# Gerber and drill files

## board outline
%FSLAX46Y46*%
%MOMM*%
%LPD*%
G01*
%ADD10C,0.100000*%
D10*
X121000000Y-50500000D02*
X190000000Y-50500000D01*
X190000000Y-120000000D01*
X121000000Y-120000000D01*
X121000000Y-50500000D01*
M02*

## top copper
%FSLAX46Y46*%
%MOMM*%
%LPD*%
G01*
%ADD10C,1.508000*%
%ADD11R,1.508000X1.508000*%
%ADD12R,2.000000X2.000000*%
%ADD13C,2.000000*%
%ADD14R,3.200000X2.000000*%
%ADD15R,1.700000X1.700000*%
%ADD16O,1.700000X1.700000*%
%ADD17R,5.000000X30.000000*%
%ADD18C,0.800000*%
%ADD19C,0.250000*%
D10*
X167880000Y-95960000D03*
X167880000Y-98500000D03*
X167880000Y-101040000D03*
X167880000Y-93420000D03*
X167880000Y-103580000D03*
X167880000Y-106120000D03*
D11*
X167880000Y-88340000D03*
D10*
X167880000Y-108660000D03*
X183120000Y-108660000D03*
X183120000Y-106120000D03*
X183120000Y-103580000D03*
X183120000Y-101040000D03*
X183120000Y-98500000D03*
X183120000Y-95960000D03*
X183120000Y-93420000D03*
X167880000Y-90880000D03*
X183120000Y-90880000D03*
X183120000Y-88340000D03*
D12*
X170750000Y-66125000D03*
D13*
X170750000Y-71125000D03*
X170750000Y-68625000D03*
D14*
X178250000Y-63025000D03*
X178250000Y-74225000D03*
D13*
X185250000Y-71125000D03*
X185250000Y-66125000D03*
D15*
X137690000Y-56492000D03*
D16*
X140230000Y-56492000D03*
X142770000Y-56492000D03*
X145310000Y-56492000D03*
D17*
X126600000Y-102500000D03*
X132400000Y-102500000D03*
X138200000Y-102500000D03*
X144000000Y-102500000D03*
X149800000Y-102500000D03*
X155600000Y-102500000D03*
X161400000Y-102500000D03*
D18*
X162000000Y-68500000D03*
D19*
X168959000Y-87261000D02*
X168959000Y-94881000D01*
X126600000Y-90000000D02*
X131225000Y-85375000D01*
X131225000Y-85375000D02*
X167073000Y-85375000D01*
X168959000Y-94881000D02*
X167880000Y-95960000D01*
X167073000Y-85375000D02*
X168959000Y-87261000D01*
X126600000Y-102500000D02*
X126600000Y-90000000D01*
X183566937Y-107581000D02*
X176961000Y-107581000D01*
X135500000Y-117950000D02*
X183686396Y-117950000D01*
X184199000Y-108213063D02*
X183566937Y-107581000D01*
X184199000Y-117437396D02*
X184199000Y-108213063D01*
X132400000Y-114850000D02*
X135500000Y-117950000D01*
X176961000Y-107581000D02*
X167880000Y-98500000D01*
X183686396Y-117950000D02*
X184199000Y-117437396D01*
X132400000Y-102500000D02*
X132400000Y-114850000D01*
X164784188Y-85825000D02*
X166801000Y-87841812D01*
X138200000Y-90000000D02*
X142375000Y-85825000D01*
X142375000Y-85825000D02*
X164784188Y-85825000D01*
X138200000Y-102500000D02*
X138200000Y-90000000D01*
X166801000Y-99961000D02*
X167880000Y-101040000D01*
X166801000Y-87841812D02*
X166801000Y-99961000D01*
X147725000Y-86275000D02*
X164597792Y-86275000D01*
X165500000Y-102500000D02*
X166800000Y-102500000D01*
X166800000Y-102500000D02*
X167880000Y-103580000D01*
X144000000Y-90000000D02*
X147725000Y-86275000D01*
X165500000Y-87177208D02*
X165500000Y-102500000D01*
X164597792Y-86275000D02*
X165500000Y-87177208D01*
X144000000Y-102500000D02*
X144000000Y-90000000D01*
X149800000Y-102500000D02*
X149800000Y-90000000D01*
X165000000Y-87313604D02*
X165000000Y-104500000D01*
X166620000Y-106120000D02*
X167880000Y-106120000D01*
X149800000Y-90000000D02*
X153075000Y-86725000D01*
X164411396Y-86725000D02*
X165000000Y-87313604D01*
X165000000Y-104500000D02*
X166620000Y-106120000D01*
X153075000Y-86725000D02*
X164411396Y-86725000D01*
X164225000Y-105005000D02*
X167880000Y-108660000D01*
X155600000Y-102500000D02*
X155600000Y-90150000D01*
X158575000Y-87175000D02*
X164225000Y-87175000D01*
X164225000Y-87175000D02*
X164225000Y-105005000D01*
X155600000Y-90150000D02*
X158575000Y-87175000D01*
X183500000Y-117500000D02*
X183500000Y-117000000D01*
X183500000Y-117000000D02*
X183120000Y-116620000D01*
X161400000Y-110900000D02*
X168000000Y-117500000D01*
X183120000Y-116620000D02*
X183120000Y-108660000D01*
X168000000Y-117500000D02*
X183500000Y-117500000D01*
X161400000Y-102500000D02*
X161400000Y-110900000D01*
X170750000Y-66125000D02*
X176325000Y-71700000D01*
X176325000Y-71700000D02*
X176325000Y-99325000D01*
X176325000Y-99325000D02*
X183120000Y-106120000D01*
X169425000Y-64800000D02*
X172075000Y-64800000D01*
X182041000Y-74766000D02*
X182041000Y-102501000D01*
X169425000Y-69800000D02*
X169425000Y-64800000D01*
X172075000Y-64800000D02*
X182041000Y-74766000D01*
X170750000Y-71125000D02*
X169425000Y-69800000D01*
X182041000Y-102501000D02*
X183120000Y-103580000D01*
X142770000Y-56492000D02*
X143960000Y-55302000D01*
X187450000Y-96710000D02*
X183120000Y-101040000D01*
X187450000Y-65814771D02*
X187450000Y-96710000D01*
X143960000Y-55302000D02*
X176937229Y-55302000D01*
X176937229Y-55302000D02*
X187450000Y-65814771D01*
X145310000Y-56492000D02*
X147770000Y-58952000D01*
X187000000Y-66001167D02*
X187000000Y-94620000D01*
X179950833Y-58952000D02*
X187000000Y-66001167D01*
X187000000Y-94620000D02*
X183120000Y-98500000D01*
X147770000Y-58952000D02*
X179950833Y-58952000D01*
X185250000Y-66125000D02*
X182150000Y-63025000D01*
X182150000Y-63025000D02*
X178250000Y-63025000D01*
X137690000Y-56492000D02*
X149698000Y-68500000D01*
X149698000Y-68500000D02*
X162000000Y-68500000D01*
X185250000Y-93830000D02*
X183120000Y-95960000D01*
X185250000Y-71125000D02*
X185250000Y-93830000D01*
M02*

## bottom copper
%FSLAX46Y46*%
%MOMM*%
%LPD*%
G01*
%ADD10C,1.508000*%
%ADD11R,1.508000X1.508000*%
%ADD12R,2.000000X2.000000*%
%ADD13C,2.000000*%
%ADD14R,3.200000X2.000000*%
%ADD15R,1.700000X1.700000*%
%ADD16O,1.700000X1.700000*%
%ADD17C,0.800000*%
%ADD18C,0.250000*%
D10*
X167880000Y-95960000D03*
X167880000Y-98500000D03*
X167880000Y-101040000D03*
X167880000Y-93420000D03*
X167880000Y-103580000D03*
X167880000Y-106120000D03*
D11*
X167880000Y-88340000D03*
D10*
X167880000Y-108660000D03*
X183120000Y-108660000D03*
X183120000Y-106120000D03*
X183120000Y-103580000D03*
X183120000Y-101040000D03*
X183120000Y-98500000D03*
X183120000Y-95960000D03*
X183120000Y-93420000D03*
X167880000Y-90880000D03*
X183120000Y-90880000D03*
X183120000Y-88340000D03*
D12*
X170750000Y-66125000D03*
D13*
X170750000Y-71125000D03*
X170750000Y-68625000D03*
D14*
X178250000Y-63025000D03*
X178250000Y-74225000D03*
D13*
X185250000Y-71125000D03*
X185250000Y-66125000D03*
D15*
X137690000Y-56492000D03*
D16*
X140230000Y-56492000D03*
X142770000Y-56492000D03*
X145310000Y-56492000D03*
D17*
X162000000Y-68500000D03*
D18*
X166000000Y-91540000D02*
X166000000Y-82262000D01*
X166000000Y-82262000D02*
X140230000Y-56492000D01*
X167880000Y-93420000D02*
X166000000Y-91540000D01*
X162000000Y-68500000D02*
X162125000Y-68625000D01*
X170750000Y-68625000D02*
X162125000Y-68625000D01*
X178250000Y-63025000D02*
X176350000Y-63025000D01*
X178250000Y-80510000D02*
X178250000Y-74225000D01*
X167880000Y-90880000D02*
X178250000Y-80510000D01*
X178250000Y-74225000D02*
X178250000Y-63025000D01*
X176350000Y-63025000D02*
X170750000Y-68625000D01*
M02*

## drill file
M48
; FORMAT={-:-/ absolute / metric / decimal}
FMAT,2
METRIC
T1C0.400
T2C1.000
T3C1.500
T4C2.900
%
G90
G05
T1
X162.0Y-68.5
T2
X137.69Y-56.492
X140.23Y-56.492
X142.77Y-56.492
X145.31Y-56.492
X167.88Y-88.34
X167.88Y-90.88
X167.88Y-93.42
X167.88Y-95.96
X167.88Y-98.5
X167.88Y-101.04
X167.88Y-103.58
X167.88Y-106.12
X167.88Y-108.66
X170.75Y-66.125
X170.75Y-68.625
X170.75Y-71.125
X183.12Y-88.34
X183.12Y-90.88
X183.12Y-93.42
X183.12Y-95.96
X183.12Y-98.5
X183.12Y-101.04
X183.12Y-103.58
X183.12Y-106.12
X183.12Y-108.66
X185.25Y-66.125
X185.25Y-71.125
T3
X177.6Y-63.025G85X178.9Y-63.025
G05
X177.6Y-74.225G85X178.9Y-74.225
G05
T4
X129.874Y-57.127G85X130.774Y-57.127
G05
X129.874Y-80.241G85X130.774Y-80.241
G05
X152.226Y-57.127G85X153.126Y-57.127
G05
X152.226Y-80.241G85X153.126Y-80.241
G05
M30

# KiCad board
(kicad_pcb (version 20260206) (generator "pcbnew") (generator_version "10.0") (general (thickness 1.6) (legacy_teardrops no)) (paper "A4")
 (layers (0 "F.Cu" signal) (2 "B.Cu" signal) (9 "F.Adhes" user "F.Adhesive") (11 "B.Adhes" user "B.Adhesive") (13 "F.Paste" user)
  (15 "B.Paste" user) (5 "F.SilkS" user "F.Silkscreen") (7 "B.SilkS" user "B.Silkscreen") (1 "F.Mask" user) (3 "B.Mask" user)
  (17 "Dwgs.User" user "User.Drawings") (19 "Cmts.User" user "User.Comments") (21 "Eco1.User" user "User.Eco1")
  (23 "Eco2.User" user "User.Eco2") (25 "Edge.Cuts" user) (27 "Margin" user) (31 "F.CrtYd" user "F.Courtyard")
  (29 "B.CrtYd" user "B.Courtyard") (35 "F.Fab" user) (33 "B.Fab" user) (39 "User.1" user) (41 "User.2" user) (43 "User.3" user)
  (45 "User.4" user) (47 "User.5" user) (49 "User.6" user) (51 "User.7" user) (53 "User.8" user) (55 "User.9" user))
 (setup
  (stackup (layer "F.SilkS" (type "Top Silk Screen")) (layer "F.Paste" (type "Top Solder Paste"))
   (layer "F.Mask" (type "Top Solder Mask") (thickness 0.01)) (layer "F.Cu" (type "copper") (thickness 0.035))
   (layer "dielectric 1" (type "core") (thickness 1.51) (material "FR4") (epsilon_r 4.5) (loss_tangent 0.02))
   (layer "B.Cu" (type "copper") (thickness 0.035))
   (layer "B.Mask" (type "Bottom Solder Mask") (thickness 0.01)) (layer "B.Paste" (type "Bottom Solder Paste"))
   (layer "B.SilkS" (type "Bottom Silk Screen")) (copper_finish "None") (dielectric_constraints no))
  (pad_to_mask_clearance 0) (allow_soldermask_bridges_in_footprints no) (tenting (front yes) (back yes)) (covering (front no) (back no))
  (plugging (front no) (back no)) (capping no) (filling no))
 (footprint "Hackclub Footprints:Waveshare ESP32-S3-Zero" (layer "F.Cu") (at 175.5 98.5)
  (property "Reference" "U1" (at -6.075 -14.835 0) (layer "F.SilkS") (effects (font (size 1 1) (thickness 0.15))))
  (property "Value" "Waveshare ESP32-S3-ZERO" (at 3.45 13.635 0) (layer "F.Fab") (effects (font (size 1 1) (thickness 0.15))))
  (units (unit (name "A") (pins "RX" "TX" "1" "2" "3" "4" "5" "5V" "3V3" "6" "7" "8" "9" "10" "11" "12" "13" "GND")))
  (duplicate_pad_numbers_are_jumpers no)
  (pad "1" thru_hole circle (at -7.62 -2.54) (size 1.508 1.508) (drill 1) (layers "*.Cu" "*.Mask") (remove_unused_layers no)
   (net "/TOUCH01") (solder_mask_margin 0.102))
  (pad "2" thru_hole circle (at -7.62 0) (size 1.508 1.508) (drill 1) (layers "*.Cu" "*.Mask") (remove_unused_layers no) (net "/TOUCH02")
   (solder_mask_margin 0.102))
  (pad "3" thru_hole circle (at -7.62 2.54) (size 1.508 1.508) (drill 1) (layers "*.Cu" "*.Mask") (remove_unused_layers no) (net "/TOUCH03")
   (solder_mask_margin 0.102))
  (pad "3V3" thru_hole circle (at -7.62 -5.08) (size 1.508 1.508) (drill 1) (layers "*.Cu" "*.Mask") (remove_unused_layers no) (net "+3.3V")
   (solder_mask_margin 0.102))
  (pad "4" thru_hole circle (at -7.62 5.08) (size 1.508 1.508) (drill 1) (layers "*.Cu" "*.Mask") (remove_unused_layers no) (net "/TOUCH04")
   (solder_mask_margin 0.102))
  (pad "5" thru_hole circle (at -7.62 7.62) (size 1.508 1.508) (drill 1) (layers "*.Cu" "*.Mask") (remove_unused_layers no) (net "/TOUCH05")
   (solder_mask_margin 0.102))
  (pad "5V" thru_hole rect (at -7.62 -10.16) (size 1.508 1.508) (drill 1) (layers "*.Cu" "*.Mask") (remove_unused_layers no) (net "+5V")
   (solder_mask_margin 0.102))
  (pad "6" thru_hole circle (at -7.62 10.16) (size 1.508 1.508) (drill 1) (layers "*.Cu" "*.Mask") (remove_unused_layers no)
   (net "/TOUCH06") (solder_mask_margin 0.102))
  (pad "7" thru_hole circle (at 7.62 10.16) (size 1.508 1.508) (drill 1) (layers "*.Cu" "*.Mask") (remove_unused_layers no) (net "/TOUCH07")
   (solder_mask_margin 0.102))
  (pad "8" thru_hole circle (at 7.62 7.62) (size 1.508 1.508) (drill 1) (layers "*.Cu" "*.Mask") (remove_unused_layers no) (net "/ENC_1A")
   (solder_mask_margin 0.102))
  (pad "9" thru_hole circle (at 7.62 5.08) (size 1.508 1.508) (drill 1) (layers "*.Cu" "*.Mask") (remove_unused_layers no) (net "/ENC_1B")
   (solder_mask_margin 0.102))
  (pad "10" thru_hole circle (at 7.62 2.54) (size 1.508 1.508) (drill 1) (layers "*.Cu" "*.Mask") (remove_unused_layers no) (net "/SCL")
   (solder_mask_margin 0.102))
  (pad "11" thru_hole circle (at 7.62 0) (size 1.508 1.508) (drill 1) (layers "*.Cu" "*.Mask") (remove_unused_layers no) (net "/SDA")
   (solder_mask_margin 0.102))
  (pad "12" thru_hole circle (at 7.62 -2.54) (size 1.508 1.508) (drill 1) (layers "*.Cu" "*.Mask") (remove_unused_layers no)
   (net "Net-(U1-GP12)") (solder_mask_margin 0.102))
  (pad "13" thru_hole circle (at 7.62 -5.08) (size 1.508 1.508) (drill 1) (layers "*.Cu" "*.Mask") (remove_unused_layers no)
   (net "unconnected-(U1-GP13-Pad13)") (solder_mask_margin 0.102))
  (pad "GND" thru_hole circle (at -7.62 -7.62) (size 1.508 1.508) (drill 1) (layers "*.Cu" "*.Mask") (remove_unused_layers no) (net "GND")
   (solder_mask_margin 0.102))
  (pad "RX" thru_hole circle (at 7.62 -7.62) (size 1.508 1.508) (drill 1) (layers "*.Cu" "*.Mask") (remove_unused_layers no)
   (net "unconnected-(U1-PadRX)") (solder_mask_margin 0.102))
  (pad "TX" thru_hole circle (at 7.62 -10.16) (size 1.508 1.508) (drill 1) (layers "*.Cu" "*.Mask") (remove_unused_layers no)
   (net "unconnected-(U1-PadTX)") (solder_mask_margin 0.102)))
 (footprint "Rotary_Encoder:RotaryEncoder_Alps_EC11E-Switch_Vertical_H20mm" (layer "F.Cu") (at 170.75 66.125)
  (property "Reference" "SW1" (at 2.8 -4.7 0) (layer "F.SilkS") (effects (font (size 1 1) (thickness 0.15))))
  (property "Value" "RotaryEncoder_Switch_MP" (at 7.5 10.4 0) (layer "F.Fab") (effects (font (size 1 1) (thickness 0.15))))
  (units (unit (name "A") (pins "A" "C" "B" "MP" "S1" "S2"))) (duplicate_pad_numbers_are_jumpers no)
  (pad "A" thru_hole rect (at 0 0) (size 2 2) (drill 1) (layers "*.Cu" "*.Mask") (remove_unused_layers no) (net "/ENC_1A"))
  (pad "B" thru_hole circle (at 0 5) (size 2 2) (drill 1) (layers "*.Cu" "*.Mask") (remove_unused_layers no) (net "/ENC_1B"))
  (pad "C" thru_hole circle (at 0 2.5) (size 2 2) (drill 1) (layers "*.Cu" "*.Mask") (remove_unused_layers no) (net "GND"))
  (pad "MP" thru_hole rect (at 7.5 -3.1) (size 3.2 2) (drill oval 2.8 1.5) (layers "*.Cu" "*.Mask") (remove_unused_layers no) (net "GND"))
  (pad "MP" thru_hole rect (at 7.5 8.1) (size 3.2 2) (drill oval 2.8 1.5) (layers "*.Cu" "*.Mask") (remove_unused_layers no) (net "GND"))
  (pad "S1" thru_hole circle (at 14.5 5) (size 2 2) (drill 1) (layers "*.Cu" "*.Mask") (remove_unused_layers no) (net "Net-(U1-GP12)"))
  (pad "S2" thru_hole circle (at 14.5 0) (size 2 2) (drill 1) (layers "*.Cu" "*.Mask") (remove_unused_layers no) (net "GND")))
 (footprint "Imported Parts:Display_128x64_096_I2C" (layer "F.Cu") (at 141.5 56.492)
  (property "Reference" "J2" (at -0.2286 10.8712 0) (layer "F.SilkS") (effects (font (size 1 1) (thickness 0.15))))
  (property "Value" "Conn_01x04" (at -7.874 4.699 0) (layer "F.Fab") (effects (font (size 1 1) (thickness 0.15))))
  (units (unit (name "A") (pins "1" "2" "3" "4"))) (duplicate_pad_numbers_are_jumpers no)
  (pad "" np_thru_hole oval (at -11.176 0.635) (size 3.8 2.9) (drill oval 3.8 2.9) (layers "*.Cu" "*.Mask"))
  (pad "" np_thru_hole oval (at -11.176 23.749) (size 3.8 2.9) (drill oval 3.8 2.9) (layers "*.Cu" "*.Mask"))
  (pad "" np_thru_hole oval (at 11.176 0.635) (size 3.8 2.9) (drill oval 3.8 2.9) (layers "*.Cu" "*.Mask"))
  (pad "" np_thru_hole oval (at 11.176 23.749) (size 3.8 2.9) (drill oval 3.8 2.9) (layers "*.Cu" "*.Mask"))
  (pad "1" thru_hole rect (at -3.81 0 90) (size 1.7 1.7) (drill 1) (layers "*.Cu" "*.Mask") (remove_unused_layers no) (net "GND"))
  (pad "2" thru_hole oval (at -1.27 0 90) (size 1.7 1.7) (drill 1) (layers "*.Cu" "*.Mask") (remove_unused_layers no) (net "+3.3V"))
  (pad "3" thru_hole oval (at 1.27 0 90) (size 1.7 1.7) (drill 1) (layers "*.Cu" "*.Mask") (remove_unused_layers no) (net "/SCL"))
  (pad "4" thru_hole oval (at 3.81 0 90) (size 1.7 1.7) (drill 1) (layers "*.Cu" "*.Mask") (remove_unused_layers no) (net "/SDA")))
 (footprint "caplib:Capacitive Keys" (layer "F.Cu") (at 125.6 98.9)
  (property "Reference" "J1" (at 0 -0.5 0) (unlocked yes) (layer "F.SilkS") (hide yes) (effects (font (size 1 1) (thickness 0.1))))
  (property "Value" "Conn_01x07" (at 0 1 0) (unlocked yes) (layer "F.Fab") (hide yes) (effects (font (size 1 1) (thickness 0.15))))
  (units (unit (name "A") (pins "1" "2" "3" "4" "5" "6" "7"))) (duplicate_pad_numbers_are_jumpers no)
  (pad "1" smd rect (at 1 3.6) (size 5 30) (layers "F.Cu" "F.Mask") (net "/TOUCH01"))
  (pad "2" smd rect (at 6.8 3.6) (size 5 30) (layers "F.Cu" "F.Mask") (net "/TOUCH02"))
  (pad "3" smd rect (at 12.6 3.6) (size 5 30) (layers "F.Cu" "F.Mask") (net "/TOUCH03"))
  (pad "4" smd rect (at 18.4 3.6) (size 5 30) (layers "F.Cu" "F.Mask") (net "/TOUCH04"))
  (pad "5" smd rect (at 24.2 3.6) (size 5 30) (layers "F.Cu" "F.Mask") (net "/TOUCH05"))
  (pad "6" smd rect (at 30 3.6) (size 5 30) (layers "F.Cu" "F.Mask") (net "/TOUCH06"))
  (pad "7" smd rect (at 35.8 3.6) (size 5 30) (layers "F.Cu" "F.Mask") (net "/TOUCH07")))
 (gr_rect (start 121 50.5) (end 190 120) (stroke (width 0.1) (type default)) (fill no) (layer "Edge.Cuts"))
 (segment (start 168.959 87.261) (end 168.959 94.881) (width 0.25) (layer "F.Cu") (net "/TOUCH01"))
 (segment (start 126.6 90) (end 131.225 85.375) (width 0.25) (layer "F.Cu") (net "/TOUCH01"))
 (segment (start 131.225 85.375) (end 167.073 85.375) (width 0.25) (layer "F.Cu") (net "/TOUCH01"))
 (segment (start 168.959 94.881) (end 167.88 95.96) (width 0.25) (layer "F.Cu") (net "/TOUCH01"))
 (segment (start 167.073 85.375) (end 168.959 87.261) (width 0.25) (layer "F.Cu") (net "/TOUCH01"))
 (segment (start 126.6 102.5) (end 126.6 90) (width 0.25) (layer "F.Cu") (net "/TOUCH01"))
 (segment (start 183.566937 107.581) (end 176.961 107.581) (width 0.25) (layer "F.Cu") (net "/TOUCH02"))
 (segment (start 135.5 117.95) (end 183.686396 117.95) (width 0.25) (layer "F.Cu") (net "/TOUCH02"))
 (segment (start 184.199 108.213063) (end 183.566937 107.581) (width 0.25) (layer "F.Cu") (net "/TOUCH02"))
 (segment (start 184.199 117.437396) (end 184.199 108.213063) (width 0.25) (layer "F.Cu") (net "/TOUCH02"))
 (segment (start 132.4 114.85) (end 135.5 117.95) (width 0.25) (layer "F.Cu") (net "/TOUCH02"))
 (segment (start 176.961 107.581) (end 167.88 98.5) (width 0.25) (layer "F.Cu") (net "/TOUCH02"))
 (segment (start 183.686396 117.95) (end 184.199 117.437396) (width 0.25) (layer "F.Cu") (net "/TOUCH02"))
 (segment (start 132.4 102.5) (end 132.4 114.85) (width 0.25) (layer "F.Cu") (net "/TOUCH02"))
 (segment (start 164.784188 85.825) (end 166.801 87.841812) (width 0.25) (layer "F.Cu") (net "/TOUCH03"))
 (segment (start 138.2 90) (end 142.375 85.825) (width 0.25) (layer "F.Cu") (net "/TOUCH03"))
 (segment (start 142.375 85.825) (end 164.784188 85.825) (width 0.25) (layer "F.Cu") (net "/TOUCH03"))
 (segment (start 138.2 102.5) (end 138.2 90) (width 0.25) (layer "F.Cu") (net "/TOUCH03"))
 (segment (start 166.801 99.961) (end 167.88 101.04) (width 0.25) (layer "F.Cu") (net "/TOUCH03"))
 (segment (start 166.801 87.841812) (end 166.801 99.961) (width 0.25) (layer "F.Cu") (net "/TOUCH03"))
 (segment (start 166 91.54) (end 166 82.262) (width 0.25) (layer "B.Cu") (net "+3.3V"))
 (segment (start 166 82.262) (end 140.23 56.492) (width 0.25) (layer "B.Cu") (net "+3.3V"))
 (segment (start 167.88 93.42) (end 166 91.54) (width 0.25) (layer "B.Cu") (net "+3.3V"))
 (segment (start 147.725 86.275) (end 164.597792 86.275) (width 0.25) (layer "F.Cu") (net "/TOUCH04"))
 (segment (start 165.5 102.5) (end 166.8 102.5) (width 0.25) (layer "F.Cu") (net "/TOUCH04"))
 (segment (start 166.8 102.5) (end 167.88 103.58) (width 0.25) (layer "F.Cu") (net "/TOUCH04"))
 (segment (start 144 90) (end 147.725 86.275) (width 0.25) (layer "F.Cu") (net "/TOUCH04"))
 (segment (start 165.5 87.177208) (end 165.5 102.5) (width 0.25) (layer "F.Cu") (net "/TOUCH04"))
 (segment (start 164.597792 86.275) (end 165.5 87.177208) (width 0.25) (layer "F.Cu") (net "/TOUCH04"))
 (segment (start 144 102.5) (end 144 90) (width 0.25) (layer "F.Cu") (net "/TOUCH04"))
 (segment (start 149.8 102.5) (end 149.8 90) (width 0.25) (layer "F.Cu") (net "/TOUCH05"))
 (segment (start 165 87.313604) (end 165 104.5) (width 0.25) (layer "F.Cu") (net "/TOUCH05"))
 (segment (start 166.62 106.12) (end 167.88 106.12) (width 0.25) (layer "F.Cu") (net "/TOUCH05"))
 (segment (start 149.8 90) (end 153.075 86.725) (width 0.25) (layer "F.Cu") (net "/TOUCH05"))
 (segment (start 164.411396 86.725) (end 165 87.313604) (width 0.25) (layer "F.Cu") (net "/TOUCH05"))
 (segment (start 165 104.5) (end 166.62 106.12) (width 0.25) (layer "F.Cu") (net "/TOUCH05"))
 (segment (start 153.075 86.725) (end 164.411396 86.725) (width 0.25) (layer "F.Cu") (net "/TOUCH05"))
 (segment (start 164.225 105.005) (end 167.88 108.66) (width 0.25) (layer "F.Cu") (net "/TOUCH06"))
 (segment (start 155.6 102.5) (end 155.6 90.15) (width 0.25) (layer "F.Cu") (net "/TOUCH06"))
 (segment (start 158.575 87.175) (end 164.225 87.175) (width 0.25) (layer "F.Cu") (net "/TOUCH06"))
 (segment (start 164.225 87.175) (end 164.225 105.005) (width 0.25) (layer "F.Cu") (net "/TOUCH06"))
 (segment (start 155.6 90.15) (end 158.575 87.175) (width 0.25) (layer "F.Cu") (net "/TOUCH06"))
 (segment (start 183.5 117.5) (end 183.5 117) (width 0.25) (layer "F.Cu") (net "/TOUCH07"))
 (segment (start 183.5 117) (end 183.12 116.62) (width 0.25) (layer "F.Cu") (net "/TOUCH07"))
 (segment (start 161.4 110.9) (end 168 117.5) (width 0.25) (layer "F.Cu") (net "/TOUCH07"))
 (segment (start 183.12 116.62) (end 183.12 108.66) (width 0.25) (layer "F.Cu") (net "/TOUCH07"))
 (segment (start 168 117.5) (end 183.5 117.5) (width 0.25) (layer "F.Cu") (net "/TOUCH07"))
 (segment (start 161.4 102.5) (end 161.4 110.9) (width 0.25) (layer "F.Cu") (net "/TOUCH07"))
 (segment (start 170.75 66.125) (end 176.325 71.7) (width 0.25) (layer "F.Cu") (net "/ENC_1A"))
 (segment (start 176.325 71.7) (end 176.325 99.325) (width 0.25) (layer "F.Cu") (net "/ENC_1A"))
 (segment (start 176.325 99.325) (end 183.12 106.12) (width 0.25) (layer "F.Cu") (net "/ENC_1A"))
 (segment (start 169.425 64.8) (end 172.075 64.8) (width 0.25) (layer "F.Cu") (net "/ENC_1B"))
 (segment (start 182.041 74.766) (end 182.041 102.501) (width 0.25) (layer "F.Cu") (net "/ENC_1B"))
 (segment (start 169.425 69.8) (end 169.425 64.8) (width 0.25) (layer "F.Cu") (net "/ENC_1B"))
 (segment (start 172.075 64.8) (end 182.041 74.766) (width 0.25) (layer "F.Cu") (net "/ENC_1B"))
 (segment (start 170.75 71.125) (end 169.425 69.8) (width 0.25) (layer "F.Cu") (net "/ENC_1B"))
 (segment (start 182.041 102.501) (end 183.12 103.58) (width 0.25) (layer "F.Cu") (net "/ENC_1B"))
 (segment (start 142.77 56.492) (end 143.96 55.302) (width 0.25) (layer "F.Cu") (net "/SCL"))
 (segment (start 187.45 96.71) (end 183.12 101.04) (width 0.25) (layer "F.Cu") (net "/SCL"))
 (segment (start 187.45 65.814771) (end 187.45 96.71) (width 0.25) (layer "F.Cu") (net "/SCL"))
 (segment (start 143.96 55.302) (end 176.937229 55.302) (width 0.25) (layer "F.Cu") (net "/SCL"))
 (segment (start 176.937229 55.302) (end 187.45 65.814771) (width 0.25) (layer "F.Cu") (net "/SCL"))
 (segment (start 145.31 56.492) (end 147.77 58.952) (width 0.25) (layer "F.Cu") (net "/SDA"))
 (segment (start 187 66.001167) (end 187 94.62) (width 0.25) (layer "F.Cu") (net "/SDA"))
 (segment (start 179.950833 58.952) (end 187 66.001167) (width 0.25) (layer "F.Cu") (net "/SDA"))
 (segment (start 187 94.62) (end 183.12 98.5) (width 0.25) (layer "F.Cu") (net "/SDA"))
 (segment (start 147.77 58.952) (end 179.950833 58.952) (width 0.25) (layer "F.Cu") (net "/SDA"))
 (segment (start 185.25 66.125) (end 182.15 63.025) (width 0.25) (layer "F.Cu") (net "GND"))
 (segment (start 182.15 63.025) (end 178.25 63.025) (width 0.25) (layer "F.Cu") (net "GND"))
 (segment (start 137.69 56.492) (end 149.698 68.5) (width 0.25) (layer "F.Cu") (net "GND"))
 (segment (start 149.698 68.5) (end 162 68.5) (width 0.25) (layer "F.Cu") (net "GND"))
 (via (at 162 68.5) (size 0.8) (drill 0.4) (layers "F.Cu" "B.Cu") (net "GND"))
 (segment (start 162 68.5) (end 162.125 68.625) (width 0.25) (layer "B.Cu") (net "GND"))
 (segment (start 170.75 68.625) (end 162.125 68.625) (width 0.25) (layer "B.Cu") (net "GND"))
 (segment (start 178.25 63.025) (end 176.35 63.025) (width 0.25) (layer "B.Cu") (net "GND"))
 (segment (start 178.25 80.51) (end 178.25 74.225) (width 0.25) (layer "B.Cu") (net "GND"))
 (segment (start 167.88 90.88) (end 178.25 80.51) (width 0.25) (layer "B.Cu") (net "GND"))
 (segment (start 178.25 74.225) (end 178.25 63.025) (width 0.25) (layer "B.Cu") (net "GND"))
 (segment (start 176.35 63.025) (end 170.75 68.625) (width 0.25) (layer "B.Cu") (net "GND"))
 (segment (start 185.25 93.83) (end 183.12 95.96) (width 0.25) (layer "F.Cu") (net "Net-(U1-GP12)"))
 (segment (start 185.25 71.125) (end 185.25 93.83) (width 0.25) (layer "F.Cu") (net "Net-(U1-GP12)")))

